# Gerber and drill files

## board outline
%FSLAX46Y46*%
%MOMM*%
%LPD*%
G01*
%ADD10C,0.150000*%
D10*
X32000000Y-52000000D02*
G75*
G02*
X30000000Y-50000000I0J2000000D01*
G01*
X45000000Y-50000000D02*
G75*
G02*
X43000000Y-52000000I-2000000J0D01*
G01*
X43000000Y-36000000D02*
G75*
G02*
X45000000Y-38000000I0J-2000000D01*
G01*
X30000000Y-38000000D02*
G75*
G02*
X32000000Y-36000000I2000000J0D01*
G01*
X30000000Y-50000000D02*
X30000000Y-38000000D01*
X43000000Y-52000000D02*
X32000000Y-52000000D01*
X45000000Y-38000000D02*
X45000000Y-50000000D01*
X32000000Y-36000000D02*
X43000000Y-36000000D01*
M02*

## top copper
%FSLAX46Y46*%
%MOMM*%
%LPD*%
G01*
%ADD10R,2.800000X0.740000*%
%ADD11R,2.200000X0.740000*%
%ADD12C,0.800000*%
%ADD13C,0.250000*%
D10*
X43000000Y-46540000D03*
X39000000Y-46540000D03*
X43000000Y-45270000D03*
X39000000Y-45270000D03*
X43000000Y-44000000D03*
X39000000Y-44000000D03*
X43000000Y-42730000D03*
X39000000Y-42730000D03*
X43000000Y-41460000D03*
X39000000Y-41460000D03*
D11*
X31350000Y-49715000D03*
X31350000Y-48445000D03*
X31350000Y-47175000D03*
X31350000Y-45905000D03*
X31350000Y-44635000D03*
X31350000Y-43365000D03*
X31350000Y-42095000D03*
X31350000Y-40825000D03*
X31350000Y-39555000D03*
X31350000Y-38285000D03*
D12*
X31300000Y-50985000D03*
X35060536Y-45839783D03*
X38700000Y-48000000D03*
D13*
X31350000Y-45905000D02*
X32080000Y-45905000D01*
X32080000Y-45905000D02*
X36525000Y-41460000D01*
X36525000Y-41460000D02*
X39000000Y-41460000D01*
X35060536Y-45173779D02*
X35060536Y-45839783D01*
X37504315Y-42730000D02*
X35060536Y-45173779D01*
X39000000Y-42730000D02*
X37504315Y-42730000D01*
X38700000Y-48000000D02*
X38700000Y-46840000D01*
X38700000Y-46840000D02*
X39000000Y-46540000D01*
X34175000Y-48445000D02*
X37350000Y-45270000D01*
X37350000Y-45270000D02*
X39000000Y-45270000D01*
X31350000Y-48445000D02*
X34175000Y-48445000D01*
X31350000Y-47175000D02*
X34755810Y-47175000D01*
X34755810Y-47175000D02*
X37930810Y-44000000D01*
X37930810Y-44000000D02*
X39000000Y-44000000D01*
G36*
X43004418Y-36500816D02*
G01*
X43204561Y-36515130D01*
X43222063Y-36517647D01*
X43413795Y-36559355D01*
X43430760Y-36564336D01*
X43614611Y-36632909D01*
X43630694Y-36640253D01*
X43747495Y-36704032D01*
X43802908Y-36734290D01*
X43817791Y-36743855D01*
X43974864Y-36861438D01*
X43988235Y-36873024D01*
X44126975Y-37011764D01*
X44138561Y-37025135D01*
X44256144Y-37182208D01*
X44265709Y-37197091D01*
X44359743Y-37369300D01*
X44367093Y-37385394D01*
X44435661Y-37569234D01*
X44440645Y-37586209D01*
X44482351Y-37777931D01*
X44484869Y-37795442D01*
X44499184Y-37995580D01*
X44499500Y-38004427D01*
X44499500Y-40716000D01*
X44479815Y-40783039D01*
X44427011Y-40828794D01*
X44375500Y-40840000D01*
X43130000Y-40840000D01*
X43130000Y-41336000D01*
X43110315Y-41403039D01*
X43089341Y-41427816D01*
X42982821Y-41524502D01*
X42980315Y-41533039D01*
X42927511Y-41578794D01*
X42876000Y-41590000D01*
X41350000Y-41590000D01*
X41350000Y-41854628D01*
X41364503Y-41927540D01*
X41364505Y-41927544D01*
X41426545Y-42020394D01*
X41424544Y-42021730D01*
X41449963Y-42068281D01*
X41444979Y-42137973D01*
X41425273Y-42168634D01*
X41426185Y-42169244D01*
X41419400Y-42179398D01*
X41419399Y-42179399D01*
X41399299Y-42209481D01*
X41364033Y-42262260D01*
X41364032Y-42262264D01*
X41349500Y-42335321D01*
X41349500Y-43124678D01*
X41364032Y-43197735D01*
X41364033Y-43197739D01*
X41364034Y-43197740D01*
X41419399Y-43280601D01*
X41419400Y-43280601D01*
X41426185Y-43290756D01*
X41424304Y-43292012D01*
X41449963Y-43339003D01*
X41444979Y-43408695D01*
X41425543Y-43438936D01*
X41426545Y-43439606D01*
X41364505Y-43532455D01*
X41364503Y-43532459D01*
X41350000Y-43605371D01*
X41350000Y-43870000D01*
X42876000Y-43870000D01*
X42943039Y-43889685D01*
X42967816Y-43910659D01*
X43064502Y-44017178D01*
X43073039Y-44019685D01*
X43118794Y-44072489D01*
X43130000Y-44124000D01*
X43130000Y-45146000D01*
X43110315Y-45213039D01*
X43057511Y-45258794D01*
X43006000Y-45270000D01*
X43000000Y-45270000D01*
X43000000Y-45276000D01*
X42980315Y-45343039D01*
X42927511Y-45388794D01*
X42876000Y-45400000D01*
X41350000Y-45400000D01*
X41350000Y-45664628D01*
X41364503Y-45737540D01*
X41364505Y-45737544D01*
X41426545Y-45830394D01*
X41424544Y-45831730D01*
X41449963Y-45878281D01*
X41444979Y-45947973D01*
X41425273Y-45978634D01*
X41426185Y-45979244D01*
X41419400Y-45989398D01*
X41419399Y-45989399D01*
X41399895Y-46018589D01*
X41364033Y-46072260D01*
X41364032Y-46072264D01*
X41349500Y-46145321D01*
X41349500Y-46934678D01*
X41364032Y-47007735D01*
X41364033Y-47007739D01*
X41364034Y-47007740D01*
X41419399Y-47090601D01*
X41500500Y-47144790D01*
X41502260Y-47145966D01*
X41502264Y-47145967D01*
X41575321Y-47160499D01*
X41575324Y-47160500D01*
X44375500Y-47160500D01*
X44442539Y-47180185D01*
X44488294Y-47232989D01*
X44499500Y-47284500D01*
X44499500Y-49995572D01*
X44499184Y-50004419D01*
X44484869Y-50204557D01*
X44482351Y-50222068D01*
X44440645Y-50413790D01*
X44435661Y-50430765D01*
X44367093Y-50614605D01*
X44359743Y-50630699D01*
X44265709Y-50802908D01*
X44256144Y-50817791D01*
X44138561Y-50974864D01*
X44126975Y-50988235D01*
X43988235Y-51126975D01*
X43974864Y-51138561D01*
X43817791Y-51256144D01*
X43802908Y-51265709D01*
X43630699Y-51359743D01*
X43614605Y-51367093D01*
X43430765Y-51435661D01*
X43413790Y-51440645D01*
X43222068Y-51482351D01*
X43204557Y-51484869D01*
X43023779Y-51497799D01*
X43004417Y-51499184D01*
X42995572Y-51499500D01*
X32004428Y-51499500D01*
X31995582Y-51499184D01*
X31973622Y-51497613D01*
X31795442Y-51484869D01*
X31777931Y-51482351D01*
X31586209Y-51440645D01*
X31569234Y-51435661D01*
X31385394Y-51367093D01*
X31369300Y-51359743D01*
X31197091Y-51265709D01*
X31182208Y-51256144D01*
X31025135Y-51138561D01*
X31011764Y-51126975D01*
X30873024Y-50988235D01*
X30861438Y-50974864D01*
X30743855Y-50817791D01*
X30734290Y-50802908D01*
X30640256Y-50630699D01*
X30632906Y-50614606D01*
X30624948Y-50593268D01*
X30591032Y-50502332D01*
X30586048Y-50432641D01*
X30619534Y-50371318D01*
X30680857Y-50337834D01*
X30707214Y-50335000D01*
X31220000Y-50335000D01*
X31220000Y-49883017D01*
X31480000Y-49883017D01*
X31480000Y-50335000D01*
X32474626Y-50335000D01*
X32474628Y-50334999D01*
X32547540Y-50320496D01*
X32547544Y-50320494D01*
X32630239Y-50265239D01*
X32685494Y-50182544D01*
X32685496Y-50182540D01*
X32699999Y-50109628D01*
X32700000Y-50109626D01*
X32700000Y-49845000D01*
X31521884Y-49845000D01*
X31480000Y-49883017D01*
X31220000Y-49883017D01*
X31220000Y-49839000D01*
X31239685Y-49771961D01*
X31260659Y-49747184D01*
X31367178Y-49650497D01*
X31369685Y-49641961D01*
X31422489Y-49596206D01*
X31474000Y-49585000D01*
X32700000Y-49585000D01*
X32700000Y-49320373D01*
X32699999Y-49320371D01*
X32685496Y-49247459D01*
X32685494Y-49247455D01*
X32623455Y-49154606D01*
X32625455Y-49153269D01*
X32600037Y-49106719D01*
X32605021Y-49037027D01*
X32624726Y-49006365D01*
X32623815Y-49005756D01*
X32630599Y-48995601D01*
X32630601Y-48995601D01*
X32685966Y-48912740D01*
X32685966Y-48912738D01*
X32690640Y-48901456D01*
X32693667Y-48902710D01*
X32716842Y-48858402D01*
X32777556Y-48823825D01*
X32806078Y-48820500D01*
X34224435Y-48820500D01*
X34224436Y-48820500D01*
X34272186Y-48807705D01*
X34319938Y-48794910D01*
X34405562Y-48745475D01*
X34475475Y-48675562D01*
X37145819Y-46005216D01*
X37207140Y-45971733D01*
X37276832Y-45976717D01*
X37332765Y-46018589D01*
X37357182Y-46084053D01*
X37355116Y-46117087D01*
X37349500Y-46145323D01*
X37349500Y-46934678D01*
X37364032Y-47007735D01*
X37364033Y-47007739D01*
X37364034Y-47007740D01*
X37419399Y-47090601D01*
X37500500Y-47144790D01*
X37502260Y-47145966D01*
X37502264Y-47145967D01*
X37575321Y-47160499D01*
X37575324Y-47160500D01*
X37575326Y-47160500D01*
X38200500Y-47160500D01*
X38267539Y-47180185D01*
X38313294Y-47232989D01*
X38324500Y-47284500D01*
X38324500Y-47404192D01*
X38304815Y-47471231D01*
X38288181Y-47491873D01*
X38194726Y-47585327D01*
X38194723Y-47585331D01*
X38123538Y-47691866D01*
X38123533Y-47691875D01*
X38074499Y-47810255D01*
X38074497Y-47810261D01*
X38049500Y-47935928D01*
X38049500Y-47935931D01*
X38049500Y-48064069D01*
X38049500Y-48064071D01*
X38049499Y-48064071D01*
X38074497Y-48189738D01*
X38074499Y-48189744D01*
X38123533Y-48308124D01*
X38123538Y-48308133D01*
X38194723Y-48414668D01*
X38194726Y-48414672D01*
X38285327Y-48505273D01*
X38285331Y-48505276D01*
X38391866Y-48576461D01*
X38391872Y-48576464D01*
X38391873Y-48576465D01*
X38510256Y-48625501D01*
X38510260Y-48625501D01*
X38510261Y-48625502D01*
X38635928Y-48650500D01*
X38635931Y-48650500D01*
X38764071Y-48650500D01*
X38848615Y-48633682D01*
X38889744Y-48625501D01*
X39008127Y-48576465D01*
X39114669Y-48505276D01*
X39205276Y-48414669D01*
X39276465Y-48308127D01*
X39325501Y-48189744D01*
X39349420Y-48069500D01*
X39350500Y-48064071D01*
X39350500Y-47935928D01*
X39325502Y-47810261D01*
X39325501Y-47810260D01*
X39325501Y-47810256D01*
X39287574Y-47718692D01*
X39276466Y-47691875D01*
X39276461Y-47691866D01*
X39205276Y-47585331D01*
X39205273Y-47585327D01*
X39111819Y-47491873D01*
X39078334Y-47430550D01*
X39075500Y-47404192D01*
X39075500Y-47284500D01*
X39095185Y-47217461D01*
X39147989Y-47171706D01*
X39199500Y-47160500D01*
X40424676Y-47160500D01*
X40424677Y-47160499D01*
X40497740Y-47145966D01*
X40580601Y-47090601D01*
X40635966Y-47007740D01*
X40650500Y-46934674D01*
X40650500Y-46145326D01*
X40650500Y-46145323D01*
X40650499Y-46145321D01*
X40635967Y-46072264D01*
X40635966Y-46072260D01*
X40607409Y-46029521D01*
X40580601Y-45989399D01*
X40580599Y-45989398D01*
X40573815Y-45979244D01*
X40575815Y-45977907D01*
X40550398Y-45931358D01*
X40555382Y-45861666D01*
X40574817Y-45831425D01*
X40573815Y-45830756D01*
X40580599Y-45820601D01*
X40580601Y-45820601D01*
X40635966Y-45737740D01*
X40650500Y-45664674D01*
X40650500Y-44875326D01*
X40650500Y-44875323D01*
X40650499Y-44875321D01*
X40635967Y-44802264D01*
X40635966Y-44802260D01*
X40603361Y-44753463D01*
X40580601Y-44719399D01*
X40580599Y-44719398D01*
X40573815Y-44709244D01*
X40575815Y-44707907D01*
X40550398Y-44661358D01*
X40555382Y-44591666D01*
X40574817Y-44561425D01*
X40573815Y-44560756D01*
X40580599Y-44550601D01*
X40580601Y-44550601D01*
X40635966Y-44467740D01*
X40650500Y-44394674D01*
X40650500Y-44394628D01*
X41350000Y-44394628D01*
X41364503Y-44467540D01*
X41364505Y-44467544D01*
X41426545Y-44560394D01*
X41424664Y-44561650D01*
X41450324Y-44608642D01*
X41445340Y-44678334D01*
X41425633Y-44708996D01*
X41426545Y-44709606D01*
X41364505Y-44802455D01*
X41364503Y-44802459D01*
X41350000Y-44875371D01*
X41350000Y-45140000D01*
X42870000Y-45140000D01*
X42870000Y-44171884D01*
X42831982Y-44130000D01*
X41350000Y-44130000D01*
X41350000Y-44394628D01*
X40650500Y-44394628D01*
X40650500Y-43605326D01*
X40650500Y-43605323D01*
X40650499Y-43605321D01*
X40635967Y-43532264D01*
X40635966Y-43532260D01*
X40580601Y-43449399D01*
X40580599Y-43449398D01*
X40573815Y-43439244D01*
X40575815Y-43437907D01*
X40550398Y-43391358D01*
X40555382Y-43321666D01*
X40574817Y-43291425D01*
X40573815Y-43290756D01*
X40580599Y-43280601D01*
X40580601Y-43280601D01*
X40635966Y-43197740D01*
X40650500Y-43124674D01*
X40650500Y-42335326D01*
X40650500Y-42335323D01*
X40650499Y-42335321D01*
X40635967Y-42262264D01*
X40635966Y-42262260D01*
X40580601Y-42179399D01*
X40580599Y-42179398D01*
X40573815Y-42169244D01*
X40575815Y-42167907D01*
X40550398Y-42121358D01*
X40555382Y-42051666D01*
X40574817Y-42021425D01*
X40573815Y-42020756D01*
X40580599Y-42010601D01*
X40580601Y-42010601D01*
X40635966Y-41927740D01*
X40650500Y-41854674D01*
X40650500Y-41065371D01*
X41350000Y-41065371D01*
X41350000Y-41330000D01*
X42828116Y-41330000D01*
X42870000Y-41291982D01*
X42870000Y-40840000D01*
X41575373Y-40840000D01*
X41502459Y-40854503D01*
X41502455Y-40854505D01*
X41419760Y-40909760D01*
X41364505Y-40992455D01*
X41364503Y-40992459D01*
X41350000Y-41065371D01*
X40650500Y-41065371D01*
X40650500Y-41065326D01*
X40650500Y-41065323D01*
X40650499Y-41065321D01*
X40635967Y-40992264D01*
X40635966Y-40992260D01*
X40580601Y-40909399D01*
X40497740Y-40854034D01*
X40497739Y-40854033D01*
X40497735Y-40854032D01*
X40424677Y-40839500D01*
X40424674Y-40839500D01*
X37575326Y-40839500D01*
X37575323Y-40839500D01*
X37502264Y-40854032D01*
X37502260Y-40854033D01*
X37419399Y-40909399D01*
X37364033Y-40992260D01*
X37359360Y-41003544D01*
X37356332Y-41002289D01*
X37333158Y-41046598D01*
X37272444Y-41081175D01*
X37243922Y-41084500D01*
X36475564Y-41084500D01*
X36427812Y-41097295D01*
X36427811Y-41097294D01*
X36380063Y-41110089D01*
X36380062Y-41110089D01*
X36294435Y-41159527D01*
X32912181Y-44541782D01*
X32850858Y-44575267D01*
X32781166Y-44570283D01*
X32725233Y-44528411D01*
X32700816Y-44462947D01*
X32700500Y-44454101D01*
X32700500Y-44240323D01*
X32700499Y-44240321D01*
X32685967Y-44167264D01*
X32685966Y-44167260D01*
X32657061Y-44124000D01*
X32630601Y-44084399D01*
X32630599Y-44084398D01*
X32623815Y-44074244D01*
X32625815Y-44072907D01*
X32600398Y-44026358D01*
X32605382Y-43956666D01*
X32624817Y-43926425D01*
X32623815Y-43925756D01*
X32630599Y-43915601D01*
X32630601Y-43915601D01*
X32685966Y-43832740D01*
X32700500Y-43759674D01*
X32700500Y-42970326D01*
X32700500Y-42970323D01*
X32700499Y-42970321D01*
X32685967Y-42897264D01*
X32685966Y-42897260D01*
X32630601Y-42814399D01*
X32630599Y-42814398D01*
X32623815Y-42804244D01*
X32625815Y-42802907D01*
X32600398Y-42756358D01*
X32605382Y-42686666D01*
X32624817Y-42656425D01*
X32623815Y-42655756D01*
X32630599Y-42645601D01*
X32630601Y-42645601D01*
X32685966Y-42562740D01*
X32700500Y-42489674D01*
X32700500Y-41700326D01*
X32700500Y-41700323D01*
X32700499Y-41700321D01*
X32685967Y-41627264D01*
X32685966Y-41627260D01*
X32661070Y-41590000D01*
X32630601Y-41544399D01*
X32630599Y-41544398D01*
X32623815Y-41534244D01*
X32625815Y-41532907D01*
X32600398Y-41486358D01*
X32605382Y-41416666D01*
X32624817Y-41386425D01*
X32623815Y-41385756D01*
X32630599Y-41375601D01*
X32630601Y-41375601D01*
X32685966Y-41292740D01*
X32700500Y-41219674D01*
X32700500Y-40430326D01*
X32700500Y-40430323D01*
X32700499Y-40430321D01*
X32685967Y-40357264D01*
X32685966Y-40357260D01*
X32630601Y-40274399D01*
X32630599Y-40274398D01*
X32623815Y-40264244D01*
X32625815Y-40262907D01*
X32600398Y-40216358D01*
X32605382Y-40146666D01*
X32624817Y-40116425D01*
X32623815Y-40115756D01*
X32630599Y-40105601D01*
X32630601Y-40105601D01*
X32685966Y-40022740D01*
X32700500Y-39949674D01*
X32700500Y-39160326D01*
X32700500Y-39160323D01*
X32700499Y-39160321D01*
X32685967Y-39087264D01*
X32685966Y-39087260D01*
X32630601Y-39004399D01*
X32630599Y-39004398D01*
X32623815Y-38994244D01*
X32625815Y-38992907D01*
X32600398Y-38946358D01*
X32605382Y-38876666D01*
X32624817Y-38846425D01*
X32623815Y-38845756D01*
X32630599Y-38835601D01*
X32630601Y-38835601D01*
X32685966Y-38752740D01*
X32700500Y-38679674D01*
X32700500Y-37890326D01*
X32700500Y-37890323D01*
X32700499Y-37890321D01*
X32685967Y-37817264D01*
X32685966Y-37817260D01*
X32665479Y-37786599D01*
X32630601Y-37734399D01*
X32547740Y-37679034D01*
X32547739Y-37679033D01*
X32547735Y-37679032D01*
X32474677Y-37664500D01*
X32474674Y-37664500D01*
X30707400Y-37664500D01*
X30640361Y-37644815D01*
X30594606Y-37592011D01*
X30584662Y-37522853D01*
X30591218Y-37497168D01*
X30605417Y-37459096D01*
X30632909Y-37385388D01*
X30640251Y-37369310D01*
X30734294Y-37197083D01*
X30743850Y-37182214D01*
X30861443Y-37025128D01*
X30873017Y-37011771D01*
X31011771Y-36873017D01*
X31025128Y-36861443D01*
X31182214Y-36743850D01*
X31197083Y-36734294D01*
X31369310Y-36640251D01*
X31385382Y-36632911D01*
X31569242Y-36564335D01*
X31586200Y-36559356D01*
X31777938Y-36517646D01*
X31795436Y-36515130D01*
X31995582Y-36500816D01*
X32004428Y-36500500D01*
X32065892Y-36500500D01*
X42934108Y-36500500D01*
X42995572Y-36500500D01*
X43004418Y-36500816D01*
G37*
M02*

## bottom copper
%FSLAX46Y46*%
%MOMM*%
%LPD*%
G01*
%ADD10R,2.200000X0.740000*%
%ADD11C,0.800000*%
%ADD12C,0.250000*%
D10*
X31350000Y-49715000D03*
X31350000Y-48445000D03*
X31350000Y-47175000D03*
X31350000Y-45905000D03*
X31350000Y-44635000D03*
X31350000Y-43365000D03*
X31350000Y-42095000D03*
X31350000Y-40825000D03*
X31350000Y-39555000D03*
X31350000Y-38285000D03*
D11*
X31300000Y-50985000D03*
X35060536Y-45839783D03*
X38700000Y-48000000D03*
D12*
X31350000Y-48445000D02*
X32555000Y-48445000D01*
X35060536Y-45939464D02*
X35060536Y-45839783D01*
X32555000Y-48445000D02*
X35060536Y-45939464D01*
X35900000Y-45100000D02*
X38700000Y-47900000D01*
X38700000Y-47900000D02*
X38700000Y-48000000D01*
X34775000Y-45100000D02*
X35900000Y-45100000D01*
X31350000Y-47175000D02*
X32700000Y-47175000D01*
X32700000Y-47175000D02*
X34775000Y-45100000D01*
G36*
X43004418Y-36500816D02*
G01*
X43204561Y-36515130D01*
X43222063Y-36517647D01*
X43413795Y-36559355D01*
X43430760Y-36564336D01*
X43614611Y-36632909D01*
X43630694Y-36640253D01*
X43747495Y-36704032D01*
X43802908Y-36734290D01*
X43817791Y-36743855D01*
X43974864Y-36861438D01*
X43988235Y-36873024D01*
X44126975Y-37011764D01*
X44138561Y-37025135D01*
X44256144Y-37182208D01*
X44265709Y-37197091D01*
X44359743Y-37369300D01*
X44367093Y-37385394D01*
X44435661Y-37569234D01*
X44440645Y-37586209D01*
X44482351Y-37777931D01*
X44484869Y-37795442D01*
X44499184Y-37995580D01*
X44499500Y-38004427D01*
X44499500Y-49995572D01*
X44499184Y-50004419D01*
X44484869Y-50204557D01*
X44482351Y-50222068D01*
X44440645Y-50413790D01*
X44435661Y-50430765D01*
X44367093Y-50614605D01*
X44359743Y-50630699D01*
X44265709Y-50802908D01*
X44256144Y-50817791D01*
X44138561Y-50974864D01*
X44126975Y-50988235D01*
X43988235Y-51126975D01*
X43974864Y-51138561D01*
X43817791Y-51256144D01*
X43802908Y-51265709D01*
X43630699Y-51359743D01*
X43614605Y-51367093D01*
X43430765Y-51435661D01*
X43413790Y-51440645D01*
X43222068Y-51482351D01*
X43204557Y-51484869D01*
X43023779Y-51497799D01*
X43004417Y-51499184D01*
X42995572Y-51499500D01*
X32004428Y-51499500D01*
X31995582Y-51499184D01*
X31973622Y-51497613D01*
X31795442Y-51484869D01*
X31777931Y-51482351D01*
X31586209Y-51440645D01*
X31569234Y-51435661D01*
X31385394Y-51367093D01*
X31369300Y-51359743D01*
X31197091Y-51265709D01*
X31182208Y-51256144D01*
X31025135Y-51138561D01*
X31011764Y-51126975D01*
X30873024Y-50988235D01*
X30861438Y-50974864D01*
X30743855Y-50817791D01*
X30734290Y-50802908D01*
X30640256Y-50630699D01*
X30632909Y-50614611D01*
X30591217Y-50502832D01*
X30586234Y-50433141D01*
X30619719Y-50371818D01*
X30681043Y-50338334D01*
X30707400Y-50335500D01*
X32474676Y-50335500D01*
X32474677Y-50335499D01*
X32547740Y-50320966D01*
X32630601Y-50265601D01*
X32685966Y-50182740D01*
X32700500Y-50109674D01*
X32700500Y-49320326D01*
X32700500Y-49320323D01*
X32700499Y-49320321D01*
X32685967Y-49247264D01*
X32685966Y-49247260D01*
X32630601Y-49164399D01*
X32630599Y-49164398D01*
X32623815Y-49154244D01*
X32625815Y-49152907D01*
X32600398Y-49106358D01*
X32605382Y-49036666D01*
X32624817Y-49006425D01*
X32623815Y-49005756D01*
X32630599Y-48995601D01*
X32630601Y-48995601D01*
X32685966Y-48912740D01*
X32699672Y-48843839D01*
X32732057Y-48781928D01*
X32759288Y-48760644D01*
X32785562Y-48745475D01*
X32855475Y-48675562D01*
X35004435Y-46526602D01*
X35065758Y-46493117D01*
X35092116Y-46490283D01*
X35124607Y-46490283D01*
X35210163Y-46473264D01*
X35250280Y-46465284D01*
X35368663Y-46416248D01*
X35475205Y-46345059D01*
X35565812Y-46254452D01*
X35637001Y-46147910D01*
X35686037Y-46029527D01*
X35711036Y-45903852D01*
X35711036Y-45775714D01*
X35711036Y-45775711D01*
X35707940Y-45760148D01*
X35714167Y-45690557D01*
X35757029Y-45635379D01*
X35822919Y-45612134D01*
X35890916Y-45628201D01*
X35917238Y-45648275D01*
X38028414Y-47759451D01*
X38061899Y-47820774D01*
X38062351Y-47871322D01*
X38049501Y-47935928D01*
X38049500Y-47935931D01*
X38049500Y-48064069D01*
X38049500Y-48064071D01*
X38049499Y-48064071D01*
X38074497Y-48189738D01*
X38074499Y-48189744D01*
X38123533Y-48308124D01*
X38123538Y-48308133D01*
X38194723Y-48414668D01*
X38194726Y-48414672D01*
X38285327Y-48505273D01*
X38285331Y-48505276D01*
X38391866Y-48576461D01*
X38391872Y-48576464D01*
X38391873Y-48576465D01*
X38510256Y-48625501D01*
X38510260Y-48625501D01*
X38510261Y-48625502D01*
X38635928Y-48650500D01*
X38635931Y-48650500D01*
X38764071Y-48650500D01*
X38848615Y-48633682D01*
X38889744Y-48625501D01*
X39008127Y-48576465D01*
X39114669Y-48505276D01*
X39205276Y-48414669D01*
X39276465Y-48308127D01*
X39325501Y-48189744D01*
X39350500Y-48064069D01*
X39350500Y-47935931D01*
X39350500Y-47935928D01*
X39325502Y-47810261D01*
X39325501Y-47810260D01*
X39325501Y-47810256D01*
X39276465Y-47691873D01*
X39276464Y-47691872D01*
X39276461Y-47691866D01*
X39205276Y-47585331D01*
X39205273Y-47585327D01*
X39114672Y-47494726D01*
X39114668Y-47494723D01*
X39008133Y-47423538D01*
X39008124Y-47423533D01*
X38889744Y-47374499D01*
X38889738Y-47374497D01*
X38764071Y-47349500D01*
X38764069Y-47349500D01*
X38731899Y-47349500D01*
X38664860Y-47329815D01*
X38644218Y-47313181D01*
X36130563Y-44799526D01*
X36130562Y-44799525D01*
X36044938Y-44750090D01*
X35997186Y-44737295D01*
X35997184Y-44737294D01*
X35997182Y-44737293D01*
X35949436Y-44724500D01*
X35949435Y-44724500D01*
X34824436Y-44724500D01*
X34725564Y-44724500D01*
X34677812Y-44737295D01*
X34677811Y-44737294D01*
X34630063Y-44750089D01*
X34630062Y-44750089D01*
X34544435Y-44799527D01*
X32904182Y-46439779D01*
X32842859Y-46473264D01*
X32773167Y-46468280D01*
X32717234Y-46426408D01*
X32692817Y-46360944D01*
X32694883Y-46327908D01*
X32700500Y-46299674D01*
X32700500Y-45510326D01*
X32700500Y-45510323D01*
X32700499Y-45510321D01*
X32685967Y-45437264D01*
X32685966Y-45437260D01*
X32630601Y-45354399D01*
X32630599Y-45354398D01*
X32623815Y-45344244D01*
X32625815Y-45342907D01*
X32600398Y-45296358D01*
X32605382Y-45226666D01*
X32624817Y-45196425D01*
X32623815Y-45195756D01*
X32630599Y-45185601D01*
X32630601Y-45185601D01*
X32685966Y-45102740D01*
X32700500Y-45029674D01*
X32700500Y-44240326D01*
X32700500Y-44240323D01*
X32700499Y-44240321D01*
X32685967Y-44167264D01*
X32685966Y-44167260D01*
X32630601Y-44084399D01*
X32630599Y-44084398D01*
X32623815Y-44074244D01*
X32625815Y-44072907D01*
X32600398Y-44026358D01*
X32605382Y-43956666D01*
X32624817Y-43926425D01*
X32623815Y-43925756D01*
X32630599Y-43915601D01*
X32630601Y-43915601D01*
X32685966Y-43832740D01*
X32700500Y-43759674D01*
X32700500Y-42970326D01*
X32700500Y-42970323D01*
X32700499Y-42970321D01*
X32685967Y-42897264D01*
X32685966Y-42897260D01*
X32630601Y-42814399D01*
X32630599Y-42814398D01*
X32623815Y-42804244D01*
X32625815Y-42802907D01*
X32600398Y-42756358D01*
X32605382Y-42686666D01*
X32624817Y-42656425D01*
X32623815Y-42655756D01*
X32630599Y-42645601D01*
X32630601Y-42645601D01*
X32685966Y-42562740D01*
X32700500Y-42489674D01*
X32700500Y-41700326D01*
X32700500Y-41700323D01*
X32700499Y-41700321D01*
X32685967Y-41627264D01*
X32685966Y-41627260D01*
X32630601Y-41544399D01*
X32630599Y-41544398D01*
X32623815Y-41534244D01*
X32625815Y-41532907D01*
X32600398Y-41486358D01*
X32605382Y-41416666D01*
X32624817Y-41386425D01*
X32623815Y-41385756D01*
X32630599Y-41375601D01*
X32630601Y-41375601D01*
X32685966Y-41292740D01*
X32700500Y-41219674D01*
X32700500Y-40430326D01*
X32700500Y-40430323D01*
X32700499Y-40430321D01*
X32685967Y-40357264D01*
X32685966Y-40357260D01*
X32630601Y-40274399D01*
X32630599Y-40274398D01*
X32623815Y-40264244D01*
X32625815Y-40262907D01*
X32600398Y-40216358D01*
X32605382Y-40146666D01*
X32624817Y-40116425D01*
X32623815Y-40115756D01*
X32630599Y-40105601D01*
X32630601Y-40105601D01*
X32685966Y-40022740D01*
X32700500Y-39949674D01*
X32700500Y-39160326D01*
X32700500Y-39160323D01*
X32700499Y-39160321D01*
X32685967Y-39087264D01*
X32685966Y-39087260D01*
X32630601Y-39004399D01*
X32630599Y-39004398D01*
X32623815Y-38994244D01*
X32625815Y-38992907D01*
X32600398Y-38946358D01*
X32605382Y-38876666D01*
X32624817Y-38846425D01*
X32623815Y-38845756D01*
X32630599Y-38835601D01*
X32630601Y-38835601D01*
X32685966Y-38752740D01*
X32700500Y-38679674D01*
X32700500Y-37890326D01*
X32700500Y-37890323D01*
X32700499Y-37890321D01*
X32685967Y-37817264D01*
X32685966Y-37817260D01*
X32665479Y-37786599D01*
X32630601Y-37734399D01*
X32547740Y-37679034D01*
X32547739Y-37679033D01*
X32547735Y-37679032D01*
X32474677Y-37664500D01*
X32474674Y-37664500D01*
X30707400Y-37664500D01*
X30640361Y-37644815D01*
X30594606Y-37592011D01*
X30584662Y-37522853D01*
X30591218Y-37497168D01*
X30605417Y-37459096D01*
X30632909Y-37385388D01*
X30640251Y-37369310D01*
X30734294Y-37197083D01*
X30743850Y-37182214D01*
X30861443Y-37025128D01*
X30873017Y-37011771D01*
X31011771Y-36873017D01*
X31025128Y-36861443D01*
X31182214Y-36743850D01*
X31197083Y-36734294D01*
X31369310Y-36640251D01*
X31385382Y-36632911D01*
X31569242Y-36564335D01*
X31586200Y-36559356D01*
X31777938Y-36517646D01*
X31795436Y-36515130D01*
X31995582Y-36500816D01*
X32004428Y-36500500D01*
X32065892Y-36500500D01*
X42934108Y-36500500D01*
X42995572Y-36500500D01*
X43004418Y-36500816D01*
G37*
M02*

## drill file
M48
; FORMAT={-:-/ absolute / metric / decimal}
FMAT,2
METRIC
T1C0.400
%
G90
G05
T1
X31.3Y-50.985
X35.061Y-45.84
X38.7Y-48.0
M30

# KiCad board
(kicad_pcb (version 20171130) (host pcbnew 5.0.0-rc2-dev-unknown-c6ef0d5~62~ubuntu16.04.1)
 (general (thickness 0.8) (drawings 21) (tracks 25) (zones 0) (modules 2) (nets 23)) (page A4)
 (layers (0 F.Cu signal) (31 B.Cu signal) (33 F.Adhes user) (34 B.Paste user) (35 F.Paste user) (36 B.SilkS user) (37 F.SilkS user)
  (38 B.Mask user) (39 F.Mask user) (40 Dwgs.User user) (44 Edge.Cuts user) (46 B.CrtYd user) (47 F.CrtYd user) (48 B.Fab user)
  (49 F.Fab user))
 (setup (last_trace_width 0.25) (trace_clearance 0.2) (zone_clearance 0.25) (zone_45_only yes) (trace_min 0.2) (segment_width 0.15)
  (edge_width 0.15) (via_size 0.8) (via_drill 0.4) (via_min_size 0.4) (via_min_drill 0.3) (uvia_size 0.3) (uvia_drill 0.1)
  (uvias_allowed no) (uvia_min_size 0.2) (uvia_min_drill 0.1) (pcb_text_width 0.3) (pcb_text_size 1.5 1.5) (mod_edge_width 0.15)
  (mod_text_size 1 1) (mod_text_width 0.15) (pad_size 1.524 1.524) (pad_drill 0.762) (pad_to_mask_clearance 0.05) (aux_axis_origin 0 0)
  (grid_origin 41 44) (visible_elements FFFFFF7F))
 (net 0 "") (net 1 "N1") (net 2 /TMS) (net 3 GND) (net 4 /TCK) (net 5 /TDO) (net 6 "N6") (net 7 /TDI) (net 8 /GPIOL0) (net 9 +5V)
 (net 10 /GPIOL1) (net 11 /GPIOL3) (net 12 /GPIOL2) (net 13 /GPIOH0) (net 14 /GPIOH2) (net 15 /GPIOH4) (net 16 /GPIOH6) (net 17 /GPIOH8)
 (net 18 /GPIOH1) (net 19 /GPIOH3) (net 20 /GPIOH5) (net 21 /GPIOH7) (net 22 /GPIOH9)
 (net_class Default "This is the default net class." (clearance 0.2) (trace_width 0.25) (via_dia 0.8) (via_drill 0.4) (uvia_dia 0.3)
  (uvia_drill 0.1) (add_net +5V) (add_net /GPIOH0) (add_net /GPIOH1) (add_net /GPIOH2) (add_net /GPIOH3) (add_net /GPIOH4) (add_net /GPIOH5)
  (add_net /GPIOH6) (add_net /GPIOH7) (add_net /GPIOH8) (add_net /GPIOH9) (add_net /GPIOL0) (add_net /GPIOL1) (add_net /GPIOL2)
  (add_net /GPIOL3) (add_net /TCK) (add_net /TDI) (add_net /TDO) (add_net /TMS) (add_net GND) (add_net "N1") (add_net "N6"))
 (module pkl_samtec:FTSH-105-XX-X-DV (layer F.Cu) (at 41 44 270)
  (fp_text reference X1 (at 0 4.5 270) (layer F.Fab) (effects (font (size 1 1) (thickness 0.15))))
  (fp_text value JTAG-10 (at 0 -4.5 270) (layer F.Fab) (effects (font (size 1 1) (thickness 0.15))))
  (pad 1 smd rect (at 2.54 -2 90) (size 0.74 2.8) (layers F.Cu F.Paste F.Mask) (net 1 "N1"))
  (pad 2 smd rect (at 2.54 2 90) (size 0.74 2.8) (layers F.Cu F.Paste F.Mask) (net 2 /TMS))
  (pad 3 smd rect (at 1.27 -2 90) (size 0.74 2.8) (layers F.Cu F.Paste F.Mask) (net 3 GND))
  (pad 4 smd rect (at 1.27 2 90) (size 0.74 2.8) (layers F.Cu F.Paste F.Mask) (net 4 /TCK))
  (pad 5 smd rect (at 0 -2 90) (size 0.74 2.8) (layers F.Cu F.Paste F.Mask) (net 3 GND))
  (pad 6 smd rect (at 0 2 90) (size 0.74 2.8) (layers F.Cu F.Paste F.Mask) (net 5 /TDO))
  (pad 7 smd rect (at -1.27 -2 90) (size 0.74 2.8) (layers F.Cu F.Paste F.Mask) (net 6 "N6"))
  (pad 8 smd rect (at -1.27 2 90) (size 0.74 2.8) (layers F.Cu F.Paste F.Mask) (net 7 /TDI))
  (pad 9 smd rect (at -2.54 -2 90) (size 0.74 2.8) (layers F.Cu F.Paste F.Mask) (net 3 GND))
  (pad 10 smd rect (at -2.54 2 90) (size 0.74 2.8) (layers F.Cu F.Paste F.Mask) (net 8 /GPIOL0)))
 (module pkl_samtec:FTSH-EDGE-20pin (layer B.Cu) (at 30 44 90)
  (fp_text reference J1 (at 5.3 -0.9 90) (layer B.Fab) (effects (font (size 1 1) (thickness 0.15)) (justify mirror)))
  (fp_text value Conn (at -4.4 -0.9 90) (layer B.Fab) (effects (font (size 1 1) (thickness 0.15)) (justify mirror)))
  (pad 1 smd rect (at -5.715 1.35 90) (size 0.74 2.2) (layers B.Cu B.Paste B.Mask) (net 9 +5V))
  (pad 2 smd rect (at -5.715 1.35 90) (size 0.74 2.2) (layers F.Cu F.Paste F.Mask) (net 3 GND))
  (pad 3 smd rect (at -4.445 1.35 90) (size 0.74 2.2) (layers B.Cu B.Paste B.Mask) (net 7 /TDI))
  (pad 5 smd rect (at -3.175 1.35 90) (size 0.74 2.2) (layers B.Cu B.Paste B.Mask) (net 2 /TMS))
  (pad 7 smd rect (at -1.905 1.35 90) (size 0.74 2.2) (layers B.Cu B.Paste B.Mask) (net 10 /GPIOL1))
  (pad 9 smd rect (at -0.635 1.35 90) (size 0.74 2.2) (layers B.Cu B.Paste B.Mask) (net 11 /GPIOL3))
  (pad 4 smd rect (at -4.445 1.35 90) (size 0.74 2.2) (layers F.Cu F.Paste F.Mask) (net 4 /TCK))
  (pad 6 smd rect (at -3.175 1.35 90) (size 0.74 2.2) (layers F.Cu F.Paste F.Mask) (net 5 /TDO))
  (pad 8 smd rect (at -1.905 1.35 90) (size 0.74 2.2) (layers F.Cu F.Paste F.Mask) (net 8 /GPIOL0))
  (pad 10 smd rect (at -0.635 1.35 90) (size 0.74 2.2) (layers F.Cu F.Paste F.Mask) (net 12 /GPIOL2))
  (pad 12 smd rect (at 0.635 1.35 90) (size 0.74 2.2) (layers F.Cu F.Paste F.Mask) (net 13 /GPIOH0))
  (pad 14 smd rect (at 1.905 1.35 90) (size 0.74 2.2) (layers F.Cu F.Paste F.Mask) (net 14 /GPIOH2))
  (pad 16 smd rect (at 3.175 1.35 90) (size 0.74 2.2) (layers F.Cu F.Paste F.Mask) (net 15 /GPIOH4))
  (pad 18 smd rect (at 4.445 1.35 90) (size 0.74 2.2) (layers F.Cu F.Paste F.Mask) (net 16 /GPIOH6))
  (pad 20 smd rect (at 5.715 1.35 90) (size 0.74 2.2) (layers F.Cu F.Paste F.Mask) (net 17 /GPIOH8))
  (pad 11 smd rect (at 0.635 1.35 90) (size 0.74 2.2) (layers B.Cu B.Paste B.Mask) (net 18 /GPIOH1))
  (pad 13 smd rect (at 1.905 1.35 90) (size 0.74 2.2) (layers B.Cu B.Paste B.Mask) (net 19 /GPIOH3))
  (pad 15 smd rect (at 3.175 1.35 90) (size 0.74 2.2) (layers B.Cu B.Paste B.Mask) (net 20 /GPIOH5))
  (pad 17 smd rect (at 4.445 1.35 90) (size 0.74 2.2) (layers B.Cu B.Paste B.Mask) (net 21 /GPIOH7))
  (pad 19 smd rect (at 5.715 1.35 90) (size 0.74 2.2) (layers B.Cu B.Paste B.Mask) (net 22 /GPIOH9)))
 (gr_arc (start 32 50) (end 30 50) (angle -90) (layer Edge.Cuts) (width 0.15))
 (gr_arc (start 43 50) (end 43 52) (angle -90) (layer Edge.Cuts) (width 0.15))
 (gr_arc (start 43 38) (end 45 38) (angle -90) (layer Edge.Cuts) (width 0.15))
 (gr_arc (start 32 38) (end 32 36) (angle -90) (layer Edge.Cuts) (width 0.15))
 (gr_line (start 30 50) (end 30 38) (layer Edge.Cuts) (width 0.15))
 (gr_line (start 43 52) (end 32 52) (layer Edge.Cuts) (width 0.15))
 (gr_line (start 45 38) (end 45 50) (layer Edge.Cuts) (width 0.15))
 (gr_line (start 32 36) (end 43 36) (layer Edge.Cuts) (width 0.15))
 (via (at 31.3 50.985) (size 0.8) (drill 0.4) (layers F.Cu B.Cu) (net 3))
 (segment (start 31.35 45.905) (end 32.08 45.905) (width 0.25) (layer F.Cu) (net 8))
 (segment (start 32.08 45.905) (end 36.525 41.46) (width 0.25) (layer F.Cu) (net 8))
 (segment (start 36.525 41.46) (end 39 41.46) (width 0.25) (layer F.Cu) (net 8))
 (segment (start 31.35 48.445) (end 32.555 48.445) (width 0.25) (layer B.Cu) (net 7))
 (segment (start 35.060536 45.939464) (end 35.060536 45.839783) (width 0.25) (layer B.Cu) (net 7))
 (segment (start 32.555 48.445) (end 35.060536 45.939464) (width 0.25) (layer B.Cu) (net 7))
 (via (at 35.060536 45.839783) (size 0.8) (drill 0.4) (layers F.Cu B.Cu) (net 7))
 (segment (start 35.060536 45.173779) (end 35.060536 45.839783) (width 0.25) (layer F.Cu) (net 7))
 (segment (start 37.504315 42.73) (end 35.060536 45.173779) (width 0.25) (layer F.Cu) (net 7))
 (segment (start 39 42.73) (end 37.504315 42.73) (width 0.25) (layer F.Cu) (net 7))
 (segment (start 38.7 48) (end 38.7 46.84) (width 0.25) (layer F.Cu) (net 2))
 (segment (start 38.7 46.84) (end 39 46.54) (width 0.25) (layer F.Cu) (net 2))
 (segment (start 35.9 45.1) (end 38.7 47.9) (width 0.25) (layer B.Cu) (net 2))
 (via (at 38.7 48) (size 0.8) (drill 0.4) (layers F.Cu B.Cu) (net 2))
 (segment (start 38.7 47.9) (end 38.7 48) (width 0.25) (layer B.Cu) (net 2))
 (segment (start 34.775 45.1) (end 35.9 45.1) (width 0.25) (layer B.Cu) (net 2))
 (segment (start 31.35 47.175) (end 32.7 47.175) (width 0.25) (layer B.Cu) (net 2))
 (segment (start 32.7 47.175) (end 34.775 45.1) (width 0.25) (layer B.Cu) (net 2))
 (segment (start 34.175 48.445) (end 37.35 45.27) (width 0.25) (layer F.Cu) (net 4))
 (segment (start 37.35 45.27) (end 39 45.27) (width 0.25) (layer F.Cu) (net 4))
 (segment (start 31.35 48.445) (end 34.175 48.445) (width 0.25) (layer F.Cu) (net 4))
 (segment (start 31.35 47.175) (end 34.75581 47.175) (width 0.25) (layer F.Cu) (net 5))
 (segment (start 34.75581 47.175) (end 37.93081 44) (width 0.25) (layer F.Cu) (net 5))
 (segment (start 37.93081 44) (end 39 44) (width 0.25) (layer F.Cu) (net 5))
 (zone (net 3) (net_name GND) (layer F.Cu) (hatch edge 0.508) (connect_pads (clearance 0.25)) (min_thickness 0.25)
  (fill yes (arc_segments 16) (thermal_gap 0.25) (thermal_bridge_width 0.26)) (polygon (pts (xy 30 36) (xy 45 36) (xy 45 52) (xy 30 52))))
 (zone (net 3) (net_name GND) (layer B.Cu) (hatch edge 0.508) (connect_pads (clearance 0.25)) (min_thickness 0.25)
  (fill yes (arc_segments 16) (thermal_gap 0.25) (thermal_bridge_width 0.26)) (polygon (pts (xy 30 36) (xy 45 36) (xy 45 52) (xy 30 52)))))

